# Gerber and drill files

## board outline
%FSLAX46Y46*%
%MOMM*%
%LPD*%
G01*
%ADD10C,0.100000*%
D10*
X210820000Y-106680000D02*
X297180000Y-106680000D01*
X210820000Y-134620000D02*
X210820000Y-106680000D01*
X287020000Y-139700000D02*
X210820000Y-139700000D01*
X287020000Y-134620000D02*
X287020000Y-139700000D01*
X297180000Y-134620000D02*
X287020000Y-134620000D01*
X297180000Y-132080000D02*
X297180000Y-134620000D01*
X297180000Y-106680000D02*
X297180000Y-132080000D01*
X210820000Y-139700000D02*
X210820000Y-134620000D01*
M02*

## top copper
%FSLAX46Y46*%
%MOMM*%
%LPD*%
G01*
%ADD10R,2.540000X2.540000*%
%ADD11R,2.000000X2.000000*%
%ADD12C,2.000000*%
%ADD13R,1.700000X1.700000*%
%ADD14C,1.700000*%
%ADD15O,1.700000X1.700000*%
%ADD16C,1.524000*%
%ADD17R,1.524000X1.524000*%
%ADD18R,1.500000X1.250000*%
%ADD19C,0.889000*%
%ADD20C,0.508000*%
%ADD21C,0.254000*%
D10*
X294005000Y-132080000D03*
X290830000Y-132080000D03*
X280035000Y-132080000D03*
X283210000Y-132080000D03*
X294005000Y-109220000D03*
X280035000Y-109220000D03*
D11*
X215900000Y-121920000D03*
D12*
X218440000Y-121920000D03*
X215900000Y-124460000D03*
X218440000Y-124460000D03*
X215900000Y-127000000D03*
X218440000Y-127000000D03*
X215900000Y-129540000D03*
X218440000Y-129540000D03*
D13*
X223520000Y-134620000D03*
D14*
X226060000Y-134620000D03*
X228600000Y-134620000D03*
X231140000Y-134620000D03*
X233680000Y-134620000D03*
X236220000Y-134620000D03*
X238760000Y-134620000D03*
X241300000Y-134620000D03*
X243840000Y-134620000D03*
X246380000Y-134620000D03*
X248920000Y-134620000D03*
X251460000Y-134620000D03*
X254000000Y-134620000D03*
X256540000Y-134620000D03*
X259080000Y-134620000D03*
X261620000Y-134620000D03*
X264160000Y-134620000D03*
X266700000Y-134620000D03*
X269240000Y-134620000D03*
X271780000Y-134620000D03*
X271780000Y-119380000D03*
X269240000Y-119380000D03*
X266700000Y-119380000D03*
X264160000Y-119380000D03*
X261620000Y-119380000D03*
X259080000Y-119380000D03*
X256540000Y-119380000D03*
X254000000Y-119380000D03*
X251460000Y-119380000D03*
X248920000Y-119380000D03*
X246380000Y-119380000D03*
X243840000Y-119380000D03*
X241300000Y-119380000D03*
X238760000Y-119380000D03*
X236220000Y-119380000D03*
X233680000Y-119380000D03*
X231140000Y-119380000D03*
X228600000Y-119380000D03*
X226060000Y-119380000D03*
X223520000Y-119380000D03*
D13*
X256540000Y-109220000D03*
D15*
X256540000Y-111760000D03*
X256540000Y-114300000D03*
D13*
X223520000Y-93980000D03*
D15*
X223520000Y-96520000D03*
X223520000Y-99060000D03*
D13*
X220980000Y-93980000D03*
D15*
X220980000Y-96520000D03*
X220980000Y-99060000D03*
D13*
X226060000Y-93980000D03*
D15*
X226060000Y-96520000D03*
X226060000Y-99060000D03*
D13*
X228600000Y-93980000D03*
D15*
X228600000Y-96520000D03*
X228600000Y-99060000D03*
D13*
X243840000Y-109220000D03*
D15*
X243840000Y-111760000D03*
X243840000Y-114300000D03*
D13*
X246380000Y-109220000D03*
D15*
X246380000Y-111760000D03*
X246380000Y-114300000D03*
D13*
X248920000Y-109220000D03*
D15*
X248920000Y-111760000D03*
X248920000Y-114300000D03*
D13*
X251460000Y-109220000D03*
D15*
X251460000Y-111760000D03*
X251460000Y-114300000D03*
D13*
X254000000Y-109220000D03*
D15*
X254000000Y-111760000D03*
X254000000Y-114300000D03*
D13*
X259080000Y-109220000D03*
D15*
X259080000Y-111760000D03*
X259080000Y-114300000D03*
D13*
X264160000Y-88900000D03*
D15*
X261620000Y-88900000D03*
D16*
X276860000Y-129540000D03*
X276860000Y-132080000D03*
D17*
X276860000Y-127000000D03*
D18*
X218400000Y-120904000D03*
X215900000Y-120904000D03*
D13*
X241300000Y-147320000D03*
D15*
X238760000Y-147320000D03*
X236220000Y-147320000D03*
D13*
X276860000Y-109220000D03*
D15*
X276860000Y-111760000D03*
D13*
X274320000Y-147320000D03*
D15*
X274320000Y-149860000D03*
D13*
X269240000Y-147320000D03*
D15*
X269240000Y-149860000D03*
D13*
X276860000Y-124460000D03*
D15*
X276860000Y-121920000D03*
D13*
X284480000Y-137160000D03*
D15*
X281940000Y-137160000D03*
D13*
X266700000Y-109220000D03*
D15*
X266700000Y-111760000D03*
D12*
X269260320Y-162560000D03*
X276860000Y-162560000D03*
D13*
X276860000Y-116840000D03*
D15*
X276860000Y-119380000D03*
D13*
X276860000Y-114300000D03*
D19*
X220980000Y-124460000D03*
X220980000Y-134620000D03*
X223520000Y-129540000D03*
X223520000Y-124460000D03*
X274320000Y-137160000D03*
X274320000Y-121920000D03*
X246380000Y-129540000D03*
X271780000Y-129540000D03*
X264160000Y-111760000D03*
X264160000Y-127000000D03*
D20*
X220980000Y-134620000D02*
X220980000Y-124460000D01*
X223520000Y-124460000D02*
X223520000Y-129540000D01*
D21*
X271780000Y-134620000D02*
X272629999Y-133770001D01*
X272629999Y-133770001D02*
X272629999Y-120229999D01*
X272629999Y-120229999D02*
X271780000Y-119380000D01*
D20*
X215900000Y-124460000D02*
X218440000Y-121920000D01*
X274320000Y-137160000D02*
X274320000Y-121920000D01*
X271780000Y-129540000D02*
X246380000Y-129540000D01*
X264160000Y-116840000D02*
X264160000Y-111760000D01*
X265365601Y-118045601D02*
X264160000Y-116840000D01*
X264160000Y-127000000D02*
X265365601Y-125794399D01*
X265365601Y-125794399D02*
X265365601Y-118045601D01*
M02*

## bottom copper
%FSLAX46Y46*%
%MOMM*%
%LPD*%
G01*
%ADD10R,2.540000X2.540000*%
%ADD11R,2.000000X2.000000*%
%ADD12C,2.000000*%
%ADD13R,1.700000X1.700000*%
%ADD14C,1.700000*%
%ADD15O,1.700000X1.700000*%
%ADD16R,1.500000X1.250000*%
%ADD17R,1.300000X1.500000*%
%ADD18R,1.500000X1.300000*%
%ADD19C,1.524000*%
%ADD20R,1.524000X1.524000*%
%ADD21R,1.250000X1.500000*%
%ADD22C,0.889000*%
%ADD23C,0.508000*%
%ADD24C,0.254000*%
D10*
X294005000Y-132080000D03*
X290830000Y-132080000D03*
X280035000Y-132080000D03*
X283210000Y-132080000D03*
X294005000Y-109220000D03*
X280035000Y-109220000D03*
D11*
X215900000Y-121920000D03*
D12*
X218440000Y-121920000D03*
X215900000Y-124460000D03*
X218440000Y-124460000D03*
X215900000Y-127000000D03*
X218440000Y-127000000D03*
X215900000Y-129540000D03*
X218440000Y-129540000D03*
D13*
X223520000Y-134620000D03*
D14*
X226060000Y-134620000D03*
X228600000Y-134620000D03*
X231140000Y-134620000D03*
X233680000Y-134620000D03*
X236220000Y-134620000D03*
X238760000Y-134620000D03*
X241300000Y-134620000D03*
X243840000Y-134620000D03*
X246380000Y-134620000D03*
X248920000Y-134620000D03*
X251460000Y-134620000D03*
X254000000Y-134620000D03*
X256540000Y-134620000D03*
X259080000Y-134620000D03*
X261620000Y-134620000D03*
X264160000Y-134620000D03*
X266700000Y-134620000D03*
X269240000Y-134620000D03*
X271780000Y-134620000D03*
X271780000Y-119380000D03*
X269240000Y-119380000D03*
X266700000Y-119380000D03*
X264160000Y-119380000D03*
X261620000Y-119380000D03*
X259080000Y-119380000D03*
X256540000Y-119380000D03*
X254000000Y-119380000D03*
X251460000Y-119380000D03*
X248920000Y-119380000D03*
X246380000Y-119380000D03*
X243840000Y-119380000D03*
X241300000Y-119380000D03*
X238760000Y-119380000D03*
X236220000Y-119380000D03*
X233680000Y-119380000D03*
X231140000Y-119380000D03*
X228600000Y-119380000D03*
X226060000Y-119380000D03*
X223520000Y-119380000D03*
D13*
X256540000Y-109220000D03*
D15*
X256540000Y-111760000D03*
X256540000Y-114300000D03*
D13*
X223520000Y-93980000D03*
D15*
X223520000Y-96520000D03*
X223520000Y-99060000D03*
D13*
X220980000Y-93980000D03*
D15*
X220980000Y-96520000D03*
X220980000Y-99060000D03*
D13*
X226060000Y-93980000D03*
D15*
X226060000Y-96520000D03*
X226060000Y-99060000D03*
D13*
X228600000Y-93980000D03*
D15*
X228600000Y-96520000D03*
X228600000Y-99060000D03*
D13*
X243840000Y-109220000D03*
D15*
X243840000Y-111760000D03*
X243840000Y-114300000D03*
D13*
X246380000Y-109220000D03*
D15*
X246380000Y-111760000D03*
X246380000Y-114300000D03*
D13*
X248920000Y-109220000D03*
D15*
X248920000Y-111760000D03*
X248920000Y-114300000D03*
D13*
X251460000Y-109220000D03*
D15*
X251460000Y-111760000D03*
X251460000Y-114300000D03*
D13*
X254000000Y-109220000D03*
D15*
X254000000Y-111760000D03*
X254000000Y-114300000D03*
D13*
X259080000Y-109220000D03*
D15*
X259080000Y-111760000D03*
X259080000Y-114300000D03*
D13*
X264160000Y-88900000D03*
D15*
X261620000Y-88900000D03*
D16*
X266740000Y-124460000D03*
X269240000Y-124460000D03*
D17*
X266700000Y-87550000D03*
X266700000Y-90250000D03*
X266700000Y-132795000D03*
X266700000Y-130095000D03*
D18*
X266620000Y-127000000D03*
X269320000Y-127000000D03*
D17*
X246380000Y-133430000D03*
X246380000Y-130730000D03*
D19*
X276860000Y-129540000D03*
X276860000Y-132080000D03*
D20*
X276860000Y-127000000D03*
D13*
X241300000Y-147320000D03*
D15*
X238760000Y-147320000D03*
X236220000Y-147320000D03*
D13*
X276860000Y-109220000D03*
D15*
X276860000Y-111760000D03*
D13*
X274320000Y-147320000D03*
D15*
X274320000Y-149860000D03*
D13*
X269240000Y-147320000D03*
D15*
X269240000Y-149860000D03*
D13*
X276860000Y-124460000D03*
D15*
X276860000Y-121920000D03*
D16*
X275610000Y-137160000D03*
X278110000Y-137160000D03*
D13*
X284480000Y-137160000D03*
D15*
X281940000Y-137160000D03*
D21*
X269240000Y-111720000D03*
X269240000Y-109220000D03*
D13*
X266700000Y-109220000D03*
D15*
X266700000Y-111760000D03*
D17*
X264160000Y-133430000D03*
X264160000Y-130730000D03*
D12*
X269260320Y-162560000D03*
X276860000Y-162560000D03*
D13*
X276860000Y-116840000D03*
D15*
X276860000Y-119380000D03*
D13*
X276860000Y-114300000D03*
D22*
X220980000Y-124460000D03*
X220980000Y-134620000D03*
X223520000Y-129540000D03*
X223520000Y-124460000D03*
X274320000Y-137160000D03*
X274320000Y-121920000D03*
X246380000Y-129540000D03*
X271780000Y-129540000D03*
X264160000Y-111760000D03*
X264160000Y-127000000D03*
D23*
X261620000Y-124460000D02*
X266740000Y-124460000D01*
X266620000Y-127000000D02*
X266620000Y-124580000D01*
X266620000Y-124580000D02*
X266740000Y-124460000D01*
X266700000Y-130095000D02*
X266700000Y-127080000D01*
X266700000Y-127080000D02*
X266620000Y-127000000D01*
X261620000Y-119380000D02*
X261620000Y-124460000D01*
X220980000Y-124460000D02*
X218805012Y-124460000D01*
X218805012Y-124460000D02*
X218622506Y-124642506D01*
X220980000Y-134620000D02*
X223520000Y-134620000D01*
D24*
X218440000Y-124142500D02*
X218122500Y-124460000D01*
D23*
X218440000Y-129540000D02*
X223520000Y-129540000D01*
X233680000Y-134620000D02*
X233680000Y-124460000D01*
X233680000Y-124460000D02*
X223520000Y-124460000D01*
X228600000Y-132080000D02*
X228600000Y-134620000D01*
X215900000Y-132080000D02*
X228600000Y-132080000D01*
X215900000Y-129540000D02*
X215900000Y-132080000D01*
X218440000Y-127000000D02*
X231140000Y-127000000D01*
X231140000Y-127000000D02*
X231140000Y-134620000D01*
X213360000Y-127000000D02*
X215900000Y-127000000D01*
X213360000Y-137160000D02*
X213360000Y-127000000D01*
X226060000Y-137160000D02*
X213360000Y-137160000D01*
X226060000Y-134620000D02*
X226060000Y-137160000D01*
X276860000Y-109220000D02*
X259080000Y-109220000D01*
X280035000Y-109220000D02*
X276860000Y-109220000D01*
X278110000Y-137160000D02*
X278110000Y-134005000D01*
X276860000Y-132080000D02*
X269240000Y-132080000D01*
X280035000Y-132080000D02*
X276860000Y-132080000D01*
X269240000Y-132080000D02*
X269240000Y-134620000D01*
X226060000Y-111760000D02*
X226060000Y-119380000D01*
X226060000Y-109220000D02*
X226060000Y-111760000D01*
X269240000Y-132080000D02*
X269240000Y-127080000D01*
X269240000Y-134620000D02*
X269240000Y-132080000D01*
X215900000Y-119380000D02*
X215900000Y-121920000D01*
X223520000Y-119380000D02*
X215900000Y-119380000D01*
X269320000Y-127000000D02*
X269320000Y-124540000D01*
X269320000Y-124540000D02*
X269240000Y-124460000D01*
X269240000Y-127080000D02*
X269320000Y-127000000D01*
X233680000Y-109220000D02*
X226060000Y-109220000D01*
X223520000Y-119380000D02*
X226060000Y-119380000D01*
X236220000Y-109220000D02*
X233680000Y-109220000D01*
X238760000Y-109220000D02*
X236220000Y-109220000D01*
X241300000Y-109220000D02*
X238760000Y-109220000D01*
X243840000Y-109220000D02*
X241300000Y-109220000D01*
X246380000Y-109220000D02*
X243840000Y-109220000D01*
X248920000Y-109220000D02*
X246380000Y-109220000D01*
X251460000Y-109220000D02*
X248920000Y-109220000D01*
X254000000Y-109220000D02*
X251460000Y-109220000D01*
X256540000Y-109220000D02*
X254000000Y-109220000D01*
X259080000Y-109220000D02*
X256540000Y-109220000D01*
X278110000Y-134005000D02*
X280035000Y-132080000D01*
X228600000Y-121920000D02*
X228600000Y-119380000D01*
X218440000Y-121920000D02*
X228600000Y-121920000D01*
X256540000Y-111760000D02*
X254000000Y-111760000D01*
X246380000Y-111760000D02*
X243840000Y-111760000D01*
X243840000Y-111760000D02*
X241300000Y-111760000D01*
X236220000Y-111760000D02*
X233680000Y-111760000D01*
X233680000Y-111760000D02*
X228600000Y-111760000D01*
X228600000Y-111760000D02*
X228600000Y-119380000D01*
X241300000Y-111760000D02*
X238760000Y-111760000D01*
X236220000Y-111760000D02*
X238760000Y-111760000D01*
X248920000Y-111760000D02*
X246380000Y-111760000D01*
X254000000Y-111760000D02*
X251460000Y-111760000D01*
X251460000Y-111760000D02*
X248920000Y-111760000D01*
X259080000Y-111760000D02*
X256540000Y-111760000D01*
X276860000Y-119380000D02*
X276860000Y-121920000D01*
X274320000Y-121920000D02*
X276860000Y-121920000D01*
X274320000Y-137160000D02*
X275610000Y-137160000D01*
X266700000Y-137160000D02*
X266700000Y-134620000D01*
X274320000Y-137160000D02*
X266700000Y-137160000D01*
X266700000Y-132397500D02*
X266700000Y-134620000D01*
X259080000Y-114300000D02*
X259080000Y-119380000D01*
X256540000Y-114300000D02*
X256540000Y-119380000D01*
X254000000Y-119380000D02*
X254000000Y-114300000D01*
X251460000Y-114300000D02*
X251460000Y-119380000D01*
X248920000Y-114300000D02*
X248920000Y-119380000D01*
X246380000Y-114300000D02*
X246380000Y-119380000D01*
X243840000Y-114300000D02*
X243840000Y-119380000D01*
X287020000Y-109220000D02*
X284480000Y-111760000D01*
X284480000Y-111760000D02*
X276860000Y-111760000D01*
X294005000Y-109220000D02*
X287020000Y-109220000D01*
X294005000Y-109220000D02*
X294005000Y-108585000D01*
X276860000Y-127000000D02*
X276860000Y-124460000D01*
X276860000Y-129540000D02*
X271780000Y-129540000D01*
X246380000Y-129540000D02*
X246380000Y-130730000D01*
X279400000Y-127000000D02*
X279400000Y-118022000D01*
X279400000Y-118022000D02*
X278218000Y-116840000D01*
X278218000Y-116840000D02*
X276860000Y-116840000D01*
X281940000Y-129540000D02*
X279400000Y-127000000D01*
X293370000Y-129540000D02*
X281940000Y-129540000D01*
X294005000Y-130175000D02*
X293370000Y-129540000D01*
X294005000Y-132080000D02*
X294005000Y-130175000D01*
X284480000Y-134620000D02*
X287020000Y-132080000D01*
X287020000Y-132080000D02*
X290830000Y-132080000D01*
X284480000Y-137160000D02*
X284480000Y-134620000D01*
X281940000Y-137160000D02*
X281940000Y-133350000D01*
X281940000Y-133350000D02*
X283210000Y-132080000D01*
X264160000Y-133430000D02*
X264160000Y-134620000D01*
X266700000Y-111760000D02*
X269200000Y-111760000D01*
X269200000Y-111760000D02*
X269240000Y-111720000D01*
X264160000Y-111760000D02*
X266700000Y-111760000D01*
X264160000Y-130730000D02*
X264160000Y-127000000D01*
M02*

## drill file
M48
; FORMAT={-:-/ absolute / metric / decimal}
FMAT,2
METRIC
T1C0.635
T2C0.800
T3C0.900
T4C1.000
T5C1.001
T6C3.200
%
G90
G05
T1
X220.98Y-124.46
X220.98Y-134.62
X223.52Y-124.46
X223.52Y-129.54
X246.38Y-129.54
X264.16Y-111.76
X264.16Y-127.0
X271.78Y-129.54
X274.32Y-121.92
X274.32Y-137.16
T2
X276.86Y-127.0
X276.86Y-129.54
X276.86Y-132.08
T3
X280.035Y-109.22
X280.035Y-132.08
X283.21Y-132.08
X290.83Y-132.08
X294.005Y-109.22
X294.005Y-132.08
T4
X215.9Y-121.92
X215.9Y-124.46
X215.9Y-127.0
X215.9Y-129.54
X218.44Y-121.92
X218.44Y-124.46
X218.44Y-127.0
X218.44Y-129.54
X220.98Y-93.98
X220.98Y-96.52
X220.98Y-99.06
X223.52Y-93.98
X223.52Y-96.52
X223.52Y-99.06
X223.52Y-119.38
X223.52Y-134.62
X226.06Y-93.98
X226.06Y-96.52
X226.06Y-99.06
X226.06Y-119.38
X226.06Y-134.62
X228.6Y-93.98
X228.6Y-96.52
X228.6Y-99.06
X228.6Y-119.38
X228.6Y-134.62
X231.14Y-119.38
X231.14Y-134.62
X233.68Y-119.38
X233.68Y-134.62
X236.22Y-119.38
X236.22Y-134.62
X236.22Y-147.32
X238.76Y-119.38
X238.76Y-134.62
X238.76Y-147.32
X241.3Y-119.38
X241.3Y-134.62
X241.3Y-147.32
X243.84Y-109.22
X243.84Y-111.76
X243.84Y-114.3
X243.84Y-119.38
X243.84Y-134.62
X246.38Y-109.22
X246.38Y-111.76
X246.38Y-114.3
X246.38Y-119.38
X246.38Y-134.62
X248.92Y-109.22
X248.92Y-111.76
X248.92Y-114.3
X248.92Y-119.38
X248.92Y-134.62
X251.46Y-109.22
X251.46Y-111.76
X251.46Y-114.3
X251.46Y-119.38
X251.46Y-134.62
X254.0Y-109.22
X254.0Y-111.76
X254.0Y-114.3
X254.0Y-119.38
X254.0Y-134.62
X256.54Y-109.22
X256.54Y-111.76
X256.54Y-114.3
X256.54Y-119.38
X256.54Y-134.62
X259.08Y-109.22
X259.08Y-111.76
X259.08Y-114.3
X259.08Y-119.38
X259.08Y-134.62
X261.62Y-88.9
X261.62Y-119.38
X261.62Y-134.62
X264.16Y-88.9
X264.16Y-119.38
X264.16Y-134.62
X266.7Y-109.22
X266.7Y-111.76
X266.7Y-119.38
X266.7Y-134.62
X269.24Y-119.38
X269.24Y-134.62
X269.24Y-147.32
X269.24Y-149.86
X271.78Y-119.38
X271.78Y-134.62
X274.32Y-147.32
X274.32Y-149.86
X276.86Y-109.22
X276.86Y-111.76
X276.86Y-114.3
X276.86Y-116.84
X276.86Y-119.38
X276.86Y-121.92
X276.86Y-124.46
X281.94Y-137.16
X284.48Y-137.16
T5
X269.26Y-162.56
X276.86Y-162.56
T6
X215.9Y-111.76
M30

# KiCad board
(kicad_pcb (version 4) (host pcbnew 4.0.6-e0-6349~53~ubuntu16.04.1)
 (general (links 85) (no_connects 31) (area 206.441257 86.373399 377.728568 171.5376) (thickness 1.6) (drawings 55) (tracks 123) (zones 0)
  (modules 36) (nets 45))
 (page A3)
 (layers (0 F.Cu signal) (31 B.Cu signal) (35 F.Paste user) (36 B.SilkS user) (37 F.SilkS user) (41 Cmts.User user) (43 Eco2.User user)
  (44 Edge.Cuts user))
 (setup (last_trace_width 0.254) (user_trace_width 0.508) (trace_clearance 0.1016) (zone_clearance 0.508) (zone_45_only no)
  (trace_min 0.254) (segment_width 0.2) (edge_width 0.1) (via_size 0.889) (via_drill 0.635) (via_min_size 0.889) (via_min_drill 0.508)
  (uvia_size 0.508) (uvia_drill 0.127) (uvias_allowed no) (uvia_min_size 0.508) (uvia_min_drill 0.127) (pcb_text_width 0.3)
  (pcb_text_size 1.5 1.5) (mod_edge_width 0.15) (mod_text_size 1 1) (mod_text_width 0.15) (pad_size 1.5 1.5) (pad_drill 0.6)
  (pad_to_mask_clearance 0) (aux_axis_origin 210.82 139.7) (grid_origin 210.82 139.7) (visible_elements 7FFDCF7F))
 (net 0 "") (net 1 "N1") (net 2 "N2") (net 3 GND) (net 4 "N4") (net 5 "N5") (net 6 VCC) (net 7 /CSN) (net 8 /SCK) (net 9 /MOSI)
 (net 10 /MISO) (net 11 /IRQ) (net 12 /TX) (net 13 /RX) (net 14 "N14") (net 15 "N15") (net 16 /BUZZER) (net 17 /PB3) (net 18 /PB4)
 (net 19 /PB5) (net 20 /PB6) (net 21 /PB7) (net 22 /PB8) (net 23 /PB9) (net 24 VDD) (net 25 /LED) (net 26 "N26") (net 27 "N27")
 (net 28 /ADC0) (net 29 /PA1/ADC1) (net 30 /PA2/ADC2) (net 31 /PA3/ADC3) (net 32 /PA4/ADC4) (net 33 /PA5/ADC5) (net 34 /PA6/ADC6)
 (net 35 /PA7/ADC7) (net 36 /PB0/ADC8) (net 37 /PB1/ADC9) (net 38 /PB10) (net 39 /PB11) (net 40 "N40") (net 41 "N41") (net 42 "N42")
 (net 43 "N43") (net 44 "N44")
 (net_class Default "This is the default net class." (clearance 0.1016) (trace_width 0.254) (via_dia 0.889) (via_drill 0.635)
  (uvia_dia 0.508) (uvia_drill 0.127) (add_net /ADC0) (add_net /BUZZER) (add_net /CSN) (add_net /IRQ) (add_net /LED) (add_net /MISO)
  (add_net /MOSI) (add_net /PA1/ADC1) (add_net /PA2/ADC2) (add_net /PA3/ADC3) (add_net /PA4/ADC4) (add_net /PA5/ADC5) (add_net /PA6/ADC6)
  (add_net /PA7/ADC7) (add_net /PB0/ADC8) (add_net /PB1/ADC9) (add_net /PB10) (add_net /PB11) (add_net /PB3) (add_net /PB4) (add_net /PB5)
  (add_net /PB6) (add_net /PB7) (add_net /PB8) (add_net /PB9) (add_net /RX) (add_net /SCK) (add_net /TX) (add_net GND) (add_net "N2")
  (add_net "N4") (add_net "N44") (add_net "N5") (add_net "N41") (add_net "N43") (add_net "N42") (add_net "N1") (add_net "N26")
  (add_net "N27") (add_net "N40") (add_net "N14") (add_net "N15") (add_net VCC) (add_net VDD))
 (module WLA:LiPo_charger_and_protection (layer F.Cu) (at 287.02 120.65 270)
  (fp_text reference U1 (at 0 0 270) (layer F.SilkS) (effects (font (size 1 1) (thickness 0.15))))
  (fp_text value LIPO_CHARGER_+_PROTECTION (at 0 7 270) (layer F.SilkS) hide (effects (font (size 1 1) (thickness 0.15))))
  (pad 3 thru_hole rect (at 11.43 -6.985 270) (size 2.54 2.54) (drill 0.9) (layers *.Cu *.Mask F.SilkS) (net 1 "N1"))
  (pad 1 thru_hole rect (at 11.43 -3.81 270) (size 2.54 2.54) (drill 0.9) (layers *.Cu *.Mask F.SilkS) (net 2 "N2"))
  (pad 4 thru_hole rect (at 11.43 6.985 270) (size 2.54 2.54) (drill 0.9) (layers *.Cu *.Mask F.SilkS) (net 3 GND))
  (pad 2 thru_hole rect (at 11.43 3.81 270) (size 2.54 2.54) (drill 0.9) (layers *.Cu *.Mask F.SilkS) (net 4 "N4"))
  (pad 5 thru_hole rect (at -11.43 -6.985 270) (size 2.54 2.54) (drill 0.9) (layers *.Cu *.Mask F.SilkS) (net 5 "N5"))
  (pad 6 thru_hole rect (at -11.43 6.985 270) (size 2.54 2.54) (drill 0.9) (layers *.Cu *.Mask F.SilkS) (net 3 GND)))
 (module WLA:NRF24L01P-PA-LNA (layer F.Cu) (at 215.9 125.73 270)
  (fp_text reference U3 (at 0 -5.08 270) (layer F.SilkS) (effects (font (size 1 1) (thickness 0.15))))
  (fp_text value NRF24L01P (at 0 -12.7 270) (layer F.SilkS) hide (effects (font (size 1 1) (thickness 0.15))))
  (pad 1 thru_hole rect (at -3.81 0 270) (size 2 2) (drill 1) (layers *.Cu *.Mask F.SilkS) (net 3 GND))
  (pad 2 thru_hole circle (at -3.81 -2.54 270) (size 2 2) (drill 1) (layers *.Cu *.Mask F.SilkS) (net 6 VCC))
  (pad 3 thru_hole circle (at -1.27 0 270) (size 2 2) (drill 1) (layers *.Cu *.Mask F.SilkS) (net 6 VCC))
  (pad 4 thru_hole circle (at -1.27 -2.54 270) (size 2 2) (drill 1) (layers *.Cu *.Mask F.SilkS) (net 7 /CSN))
  (pad 5 thru_hole circle (at 1.27 0 270) (size 2 2) (drill 1) (layers *.Cu *.Mask F.SilkS) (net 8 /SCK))
  (pad 6 thru_hole circle (at 1.27 -2.54 270) (size 2 2) (drill 1) (layers *.Cu *.Mask F.SilkS) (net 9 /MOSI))
  (pad 7 thru_hole circle (at 3.81 0 270) (size 2 2) (drill 1) (layers *.Cu *.Mask F.SilkS) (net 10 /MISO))
  (pad 8 thru_hole circle (at 3.81 -2.54 270) (size 2 2) (drill 1) (layers *.Cu *.Mask F.SilkS) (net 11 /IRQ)))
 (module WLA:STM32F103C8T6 (layer F.Cu) (at 247.65 127)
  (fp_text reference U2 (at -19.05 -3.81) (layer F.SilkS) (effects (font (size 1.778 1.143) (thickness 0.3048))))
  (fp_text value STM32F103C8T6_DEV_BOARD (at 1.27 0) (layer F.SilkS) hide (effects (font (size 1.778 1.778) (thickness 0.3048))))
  (pad 1 thru_hole rect (at -24.13 7.62) (size 1.7 1.7) (drill 1) (layers *.Cu *.Mask F.SilkS) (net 7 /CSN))
  (pad 2 thru_hole circle (at -21.59 7.62) (size 1.7 1.7) (drill 1) (layers *.Cu *.Mask F.SilkS) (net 8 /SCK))
  (pad 3 thru_hole circle (at -19.05 7.62) (size 1.7 1.7) (drill 1) (layers *.Cu *.Mask F.SilkS) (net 10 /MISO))
  (pad 4 thru_hole circle (at -16.51 7.62) (size 1.7 1.7) (drill 1) (layers *.Cu *.Mask F.SilkS) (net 9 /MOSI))
  (pad 5 thru_hole circle (at -13.97 7.62) (size 1.7 1.7) (drill 1) (layers *.Cu *.Mask F.SilkS) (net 11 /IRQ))
  (pad 6 thru_hole circle (at -11.43 7.62) (size 1.7 1.7) (drill 1) (layers *.Cu *.Mask F.SilkS) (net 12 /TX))
  (pad 7 thru_hole circle (at -8.89 7.62) (size 1.7 1.7) (drill 1) (layers *.Cu *.Mask F.SilkS) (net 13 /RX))
  (pad 8 thru_hole circle (at -6.35 7.62) (size 1.7 1.7) (drill 1) (layers *.Cu *.Mask F.SilkS) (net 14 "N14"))
  (pad 9 thru_hole circle (at -3.81 7.62) (size 1.7 1.7) (drill 1) (layers *.Cu *.Mask F.SilkS) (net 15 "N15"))
  (pad 10 thru_hole circle (at -1.27 7.62) (size 1.7 1.7) (drill 1) (layers *.Cu *.Mask F.SilkS) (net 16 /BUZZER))
  (pad 11 thru_hole circle (at 1.27 7.62) (size 1.7 1.7) (drill 1) (layers *.Cu *.Mask F.SilkS) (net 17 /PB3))
  (pad 12 thru_hole circle (at 3.81 7.62) (size 1.7 1.7) (drill 1) (layers *.Cu *.Mask F.SilkS) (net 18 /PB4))
  (pad 13 thru_hole circle (at 6.35 7.62) (size 1.7 1.7) (drill 1) (layers *.Cu *.Mask F.SilkS) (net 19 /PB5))
  (pad 14 thru_hole circle (at 8.89 7.62) (size 1.7 1.7) (drill 1) (layers *.Cu *.Mask F.SilkS) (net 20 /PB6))
  (pad 15 thru_hole circle (at 11.43 7.62) (size 1.7 1.7) (drill 1) (layers *.Cu *.Mask F.SilkS) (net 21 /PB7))
  (pad 16 thru_hole circle (at 13.97 7.62) (size 1.7 1.7) (drill 1) (layers *.Cu *.Mask F.SilkS) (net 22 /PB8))
  (pad 17 thru_hole circle (at 16.51 7.62) (size 1.7 1.7) (drill 1) (layers *.Cu *.Mask F.SilkS) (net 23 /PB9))
  (pad 18 thru_hole circle (at 19.05 7.62) (size 1.7 1.7) (drill 1) (layers *.Cu *.Mask F.SilkS) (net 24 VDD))
  (pad 19 thru_hole circle (at 21.59 7.62) (size 1.7 1.7) (drill 1) (layers *.Cu *.Mask F.SilkS) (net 3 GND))
  (pad 20 thru_hole circle (at 24.13 7.62) (size 1.7 1.7) (drill 1) (layers *.Cu *.Mask F.SilkS) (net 6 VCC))
  (pad 21 thru_hole circle (at 24.13 -7.62) (size 1.7 1.7) (drill 1) (layers *.Cu *.Mask F.SilkS) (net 6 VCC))
  (pad 22 thru_hole circle (at 21.59 -7.62) (size 1.7 1.7) (drill 1) (layers *.Cu *.Mask F.SilkS) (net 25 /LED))
  (pad 23 thru_hole circle (at 19.05 -7.62) (size 1.7 1.7) (drill 1) (layers *.Cu *.Mask F.SilkS) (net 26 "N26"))
  (pad 24 thru_hole circle (at 16.51 -7.62) (size 1.7 1.7) (drill 1) (layers *.Cu *.Mask F.SilkS) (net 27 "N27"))
  (pad 25 thru_hole circle (at 13.97 -7.62) (size 1.7 1.7) (drill 1) (layers *.Cu *.Mask F.SilkS) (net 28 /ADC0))
  (pad 26 thru_hole circle (at 11.43 -7.62) (size 1.7 1.7) (drill 1) (layers *.Cu *.Mask F.SilkS) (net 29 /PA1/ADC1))
  (pad 27 thru_hole circle (at 8.89 -7.62) (size 1.7 1.7) (drill 1) (layers *.Cu *.Mask F.SilkS) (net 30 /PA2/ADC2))
  (pad 28 thru_hole circle (at 6.35 -7.62) (size 1.7 1.7) (drill 1) (layers *.Cu *.Mask F.SilkS) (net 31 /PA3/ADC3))
  (pad 29 thru_hole circle (at 3.81 -7.62) (size 1.7 1.7) (drill 1) (layers *.Cu *.Mask F.SilkS) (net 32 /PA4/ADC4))
  (pad 30 thru_hole circle (at 1.27 -7.62) (size 1.7 1.7) (drill 1) (layers *.Cu *.Mask F.SilkS) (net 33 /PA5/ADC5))
  (pad 31 thru_hole circle (at -1.27 -7.62) (size 1.7 1.7) (drill 1) (layers *.Cu *.Mask F.SilkS) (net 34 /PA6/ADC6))
  (pad 32 thru_hole circle (at -3.81 -7.62) (size 1.7 1.7) (drill 1) (layers *.Cu *.Mask F.SilkS) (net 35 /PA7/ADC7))
  (pad 33 thru_hole circle (at -6.35 -7.62) (size 1.7 1.7) (drill 1) (layers *.Cu *.Mask F.SilkS) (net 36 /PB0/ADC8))
  (pad 34 thru_hole circle (at -8.89 -7.62) (size 1.7 1.7) (drill 1) (layers *.Cu *.Mask F.SilkS) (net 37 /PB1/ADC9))
  (pad 35 thru_hole circle (at -11.43 -7.62) (size 1.7 1.7) (drill 1) (layers *.Cu *.Mask F.SilkS) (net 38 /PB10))
  (pad 36 thru_hole circle (at -13.97 -7.62) (size 1.7 1.7) (drill 1) (layers *.Cu *.Mask F.SilkS) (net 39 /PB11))
  (pad 37 thru_hole circle (at -16.51 -7.62) (size 1.7 1.7) (drill 1) (layers *.Cu *.Mask F.SilkS) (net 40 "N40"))
  (pad 38 thru_hole circle (at -19.05 -7.62) (size 1.7 1.7) (drill 1) (layers *.Cu *.Mask F.SilkS) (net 6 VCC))
  (pad 39 thru_hole circle (at -21.59 -7.62) (size 1.7 1.7) (drill 1) (layers *.Cu *.Mask F.SilkS) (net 3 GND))
  (pad 40 thru_hole circle (at -24.13 -7.62) (size 1.7 1.7) (drill 1) (layers *.Cu *.Mask F.SilkS) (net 3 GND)))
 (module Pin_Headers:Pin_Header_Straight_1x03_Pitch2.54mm (layer F.Cu) (at 256.54 109.22)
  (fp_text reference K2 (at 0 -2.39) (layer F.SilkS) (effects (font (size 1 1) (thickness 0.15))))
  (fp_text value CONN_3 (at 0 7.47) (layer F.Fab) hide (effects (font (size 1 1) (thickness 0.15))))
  (pad 1 thru_hole rect (at 0 0) (size 1.7 1.7) (drill 1) (layers *.Cu *.Mask) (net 3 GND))
  (pad 2 thru_hole oval (at 0 2.54) (size 1.7 1.7) (drill 1) (layers *.Cu *.Mask) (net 6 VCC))
  (pad 3 thru_hole oval (at 0 5.08) (size 1.7 1.7) (drill 1) (layers *.Cu *.Mask) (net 30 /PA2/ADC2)))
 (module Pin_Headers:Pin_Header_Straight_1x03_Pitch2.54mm (layer F.Cu) (at 223.52 93.98)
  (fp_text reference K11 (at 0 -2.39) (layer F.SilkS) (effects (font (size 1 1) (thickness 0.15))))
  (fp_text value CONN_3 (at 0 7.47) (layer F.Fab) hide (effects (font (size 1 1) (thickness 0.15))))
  (pad 1 thru_hole rect (at 0 0) (size 1.7 1.7) (drill 1) (layers *.Cu *.Mask) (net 3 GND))
  (pad 2 thru_hole oval (at 0 2.54) (size 1.7 1.7) (drill 1) (layers *.Cu *.Mask) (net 6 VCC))
  (pad 3 thru_hole oval (at 0 5.08) (size 1.7 1.7) (drill 1) (layers *.Cu *.Mask) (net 38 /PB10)))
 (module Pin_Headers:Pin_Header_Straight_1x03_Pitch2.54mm (layer F.Cu) (at 220.98 93.98)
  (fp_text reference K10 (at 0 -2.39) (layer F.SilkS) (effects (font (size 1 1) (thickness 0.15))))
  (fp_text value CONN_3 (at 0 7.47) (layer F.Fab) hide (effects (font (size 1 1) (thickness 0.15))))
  (pad 1 thru_hole rect (at 0 0) (size 1.7 1.7) (drill 1) (layers *.Cu *.Mask) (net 3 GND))
  (pad 2 thru_hole oval (at 0 2.54) (size 1.7 1.7) (drill 1) (layers *.Cu *.Mask) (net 6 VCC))
  (pad 3 thru_hole oval (at 0 5.08) (size 1.7 1.7) (drill 1) (layers *.Cu *.Mask) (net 39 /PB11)))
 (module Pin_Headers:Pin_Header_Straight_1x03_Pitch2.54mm (layer F.Cu) (at 226.06 93.98)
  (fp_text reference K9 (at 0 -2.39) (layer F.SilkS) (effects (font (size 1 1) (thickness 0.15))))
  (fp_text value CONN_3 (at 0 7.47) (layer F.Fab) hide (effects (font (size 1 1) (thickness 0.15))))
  (pad 1 thru_hole rect (at 0 0) (size 1.7 1.7) (drill 1) (layers *.Cu *.Mask) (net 3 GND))
  (pad 2 thru_hole oval (at 0 2.54) (size 1.7 1.7) (drill 1) (layers *.Cu *.Mask) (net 6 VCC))
  (pad 3 thru_hole oval (at 0 5.08) (size 1.7 1.7) (drill 1) (layers *.Cu *.Mask) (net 37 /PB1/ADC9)))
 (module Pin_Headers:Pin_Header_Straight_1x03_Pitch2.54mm (layer F.Cu) (at 228.6 93.98)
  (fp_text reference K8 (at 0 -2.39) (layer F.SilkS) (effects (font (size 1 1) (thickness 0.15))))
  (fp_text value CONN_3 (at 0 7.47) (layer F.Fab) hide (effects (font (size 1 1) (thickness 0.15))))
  (pad 1 thru_hole rect (at 0 0) (size 1.7 1.7) (drill 1) (layers *.Cu *.Mask) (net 3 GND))
  (pad 2 thru_hole oval (at 0 2.54) (size 1.7 1.7) (drill 1) (layers *.Cu *.Mask) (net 6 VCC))
  (pad 3 thru_hole oval (at 0 5.08) (size 1.7 1.7) (drill 1) (layers *.Cu *.Mask) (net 36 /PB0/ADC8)))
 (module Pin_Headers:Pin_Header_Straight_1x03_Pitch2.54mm (layer F.Cu) (at 243.84 109.22)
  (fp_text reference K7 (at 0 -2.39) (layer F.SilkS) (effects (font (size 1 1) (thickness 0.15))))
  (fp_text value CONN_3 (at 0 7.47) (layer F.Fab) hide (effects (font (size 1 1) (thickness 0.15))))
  (pad 1 thru_hole rect (at 0 0) (size 1.7 1.7) (drill 1) (layers *.Cu *.Mask) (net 3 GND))
  (pad 2 thru_hole oval (at 0 2.54) (size 1.7 1.7) (drill 1) (layers *.Cu *.Mask) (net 6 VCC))
  (pad 3 thru_hole oval (at 0 5.08) (size 1.7 1.7) (drill 1) (layers *.Cu *.Mask) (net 35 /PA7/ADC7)))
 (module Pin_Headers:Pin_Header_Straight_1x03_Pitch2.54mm (layer F.Cu) (at 246.38 109.22)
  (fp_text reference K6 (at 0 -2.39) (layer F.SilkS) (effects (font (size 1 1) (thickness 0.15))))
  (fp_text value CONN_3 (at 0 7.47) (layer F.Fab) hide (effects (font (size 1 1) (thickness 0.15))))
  (pad 1 thru_hole rect (at 0 0) (size 1.7 1.7) (drill 1) (layers *.Cu *.Mask) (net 3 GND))
  (pad 2 thru_hole oval (at 0 2.54) (size 1.7 1.7) (drill 1) (layers *.Cu *.Mask) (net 6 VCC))
  (pad 3 thru_hole oval (at 0 5.08) (size 1.7 1.7) (drill 1) (layers *.Cu *.Mask) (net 34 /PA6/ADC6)))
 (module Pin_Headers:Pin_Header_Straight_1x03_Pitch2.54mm (layer F.Cu) (at 248.92 109.22)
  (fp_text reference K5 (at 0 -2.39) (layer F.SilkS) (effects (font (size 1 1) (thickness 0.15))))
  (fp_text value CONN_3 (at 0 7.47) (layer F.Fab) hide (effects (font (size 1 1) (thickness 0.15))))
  (pad 1 thru_hole rect (at 0 0) (size 1.7 1.7) (drill 1) (layers *.Cu *.Mask) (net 3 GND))
  (pad 2 thru_hole oval (at 0 2.54) (size 1.7 1.7) (drill 1) (layers *.Cu *.Mask) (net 6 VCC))
  (pad 3 thru_hole oval (at 0 5.08) (size 1.7 1.7) (drill 1) (layers *.Cu *.Mask) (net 33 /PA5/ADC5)))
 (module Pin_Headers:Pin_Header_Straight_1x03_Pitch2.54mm (layer F.Cu) (at 251.46 109.22)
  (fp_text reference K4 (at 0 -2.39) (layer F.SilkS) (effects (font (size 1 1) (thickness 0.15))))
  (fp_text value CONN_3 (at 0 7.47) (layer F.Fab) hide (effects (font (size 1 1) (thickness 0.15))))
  (pad 1 thru_hole rect (at 0 0) (size 1.7 1.7) (drill 1) (layers *.Cu *.Mask) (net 3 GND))
  (pad 2 thru_hole oval (at 0 2.54) (size 1.7 1.7) (drill 1) (layers *.Cu *.Mask) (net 6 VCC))
  (pad 3 thru_hole oval (at 0 5.08) (size 1.7 1.7) (drill 1) (layers *.Cu *.Mask) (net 32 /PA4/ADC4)))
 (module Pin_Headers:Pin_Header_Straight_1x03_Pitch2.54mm (layer F.Cu) (at 254 109.22)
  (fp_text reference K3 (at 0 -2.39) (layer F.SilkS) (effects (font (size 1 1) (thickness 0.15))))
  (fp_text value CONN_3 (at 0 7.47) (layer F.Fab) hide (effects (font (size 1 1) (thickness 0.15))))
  (pad 1 thru_hole rect (at 0 0) (size 1.7 1.7) (drill 1) (layers *.Cu *.Mask) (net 3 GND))
  (pad 2 thru_hole oval (at 0 2.54) (size 1.7 1.7) (drill 1) (layers *.Cu *.Mask) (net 6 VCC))
  (pad 3 thru_hole oval (at 0 5.08) (size 1.7 1.7) (drill 1) (layers *.Cu *.Mask) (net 31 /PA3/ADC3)))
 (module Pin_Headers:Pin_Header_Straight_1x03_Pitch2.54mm (layer F.Cu) (at 259.08 109.22)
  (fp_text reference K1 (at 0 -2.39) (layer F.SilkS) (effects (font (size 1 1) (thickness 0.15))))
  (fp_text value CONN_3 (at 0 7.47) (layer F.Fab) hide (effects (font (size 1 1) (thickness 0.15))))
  (pad 1 thru_hole rect (at 0 0) (size 1.7 1.7) (drill 1) (layers *.Cu *.Mask) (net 3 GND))
  (pad 2 thru_hole oval (at 0 2.54) (size 1.7 1.7) (drill 1) (layers *.Cu *.Mask) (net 6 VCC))
  (pad 3 thru_hole oval (at 0 5.08) (size 1.7 1.7) (drill 1) (layers *.Cu *.Mask) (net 29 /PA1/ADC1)))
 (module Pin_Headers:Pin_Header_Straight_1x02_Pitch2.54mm (layer F.Cu) (at 264.16 88.9 270)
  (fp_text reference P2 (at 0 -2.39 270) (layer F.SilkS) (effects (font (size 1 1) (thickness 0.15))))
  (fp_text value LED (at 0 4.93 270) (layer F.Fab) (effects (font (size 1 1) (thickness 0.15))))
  (pad 1 thru_hole rect (at 0 0 270) (size 1.7 1.7) (drill 1) (layers *.Cu *.Mask) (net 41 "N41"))
  (pad 2 thru_hole oval (at 0 2.54 270) (size 1.7 1.7) (drill 1) (layers *.Cu *.Mask) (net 6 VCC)))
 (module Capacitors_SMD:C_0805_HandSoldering (layer B.Cu) (at 267.99 124.46)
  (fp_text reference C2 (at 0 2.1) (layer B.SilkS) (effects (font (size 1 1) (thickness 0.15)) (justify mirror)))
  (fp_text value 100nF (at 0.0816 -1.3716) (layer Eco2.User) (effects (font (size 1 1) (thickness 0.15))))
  (pad 1 smd rect (at -1.25 0) (size 1.5 1.25) (layers B.Cu) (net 28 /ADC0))
  (pad 2 smd rect (at 1.25 0) (size 1.5 1.25) (layers B.Cu) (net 3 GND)))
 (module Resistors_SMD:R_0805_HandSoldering (layer B.Cu) (at 266.7 88.9 270)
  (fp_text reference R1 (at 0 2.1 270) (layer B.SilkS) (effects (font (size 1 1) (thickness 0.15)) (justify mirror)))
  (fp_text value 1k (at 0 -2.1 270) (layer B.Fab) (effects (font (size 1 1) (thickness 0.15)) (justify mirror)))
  (pad 1 smd rect (at -1.35 0 270) (size 1.5 1.3) (layers B.Cu) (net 41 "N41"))
  (pad 2 smd rect (at 1.35 0 270) (size 1.5 1.3) (layers B.Cu) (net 25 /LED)))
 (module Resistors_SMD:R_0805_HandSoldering (layer B.Cu) (at 266.7 131.445 90)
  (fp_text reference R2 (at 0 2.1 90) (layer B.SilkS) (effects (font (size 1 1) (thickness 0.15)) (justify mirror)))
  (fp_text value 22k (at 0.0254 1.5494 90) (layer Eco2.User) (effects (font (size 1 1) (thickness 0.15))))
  (pad 1 smd rect (at -1.35 0 90) (size 1.5 1.3) (layers B.Cu) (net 24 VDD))
  (pad 2 smd rect (at 1.35 0 90) (size 1.5 1.3) (layers B.Cu) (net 28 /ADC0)))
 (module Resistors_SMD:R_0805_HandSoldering (layer B.Cu) (at 267.97 127)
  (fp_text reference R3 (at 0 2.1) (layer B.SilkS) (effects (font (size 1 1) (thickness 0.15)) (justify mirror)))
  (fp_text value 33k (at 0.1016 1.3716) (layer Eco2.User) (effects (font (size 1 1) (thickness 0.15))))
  (pad 1 smd rect (at -1.35 0) (size 1.5 1.3) (layers B.Cu) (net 28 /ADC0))
  (pad 2 smd rect (at 1.35 0) (size 1.5 1.3) (layers B.Cu) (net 3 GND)))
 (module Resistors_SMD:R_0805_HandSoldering (layer B.Cu) (at 246.38 132.08 90)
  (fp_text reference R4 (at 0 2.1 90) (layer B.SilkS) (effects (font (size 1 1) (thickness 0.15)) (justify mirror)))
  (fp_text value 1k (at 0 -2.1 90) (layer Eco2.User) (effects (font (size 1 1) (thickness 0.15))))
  (pad 1 smd rect (at -1.35 0 90) (size 1.5 1.3) (layers B.Cu) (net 16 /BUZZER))
  (pad 2 smd rect (at 1.35 0 90) (size 1.5 1.3) (layers B.Cu) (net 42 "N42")))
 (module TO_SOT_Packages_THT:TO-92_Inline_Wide (layer F.Cu) (at 276.86 127 270)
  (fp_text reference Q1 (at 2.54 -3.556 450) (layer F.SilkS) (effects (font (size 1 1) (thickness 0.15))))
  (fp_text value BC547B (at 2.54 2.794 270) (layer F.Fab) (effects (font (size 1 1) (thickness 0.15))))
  (pad 2 thru_hole circle (at 2.54 0) (size 1.524 1.524) (drill 0.8) (layers *.Cu *.Mask) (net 42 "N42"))
  (pad 3 thru_hole circle (at 5.08 0) (size 1.524 1.524) (drill 0.8) (layers *.Cu *.Mask) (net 3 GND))
  (pad 1 thru_hole rect (at 0 0) (size 1.524 1.524) (drill 0.8) (layers *.Cu *.Mask) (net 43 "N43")))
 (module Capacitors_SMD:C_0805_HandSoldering (layer F.Cu) (at 217.15 120.904 180)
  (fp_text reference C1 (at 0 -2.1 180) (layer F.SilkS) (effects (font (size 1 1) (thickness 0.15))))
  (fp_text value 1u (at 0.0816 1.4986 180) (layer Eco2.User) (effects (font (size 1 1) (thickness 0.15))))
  (pad 1 smd rect (at -1.25 0 180) (size 1.5 1.25) (layers F.Cu F.Paste) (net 6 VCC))
  (pad 2 smd rect (at 1.25 0 180) (size 1.5 1.25) (layers F.Cu F.Paste) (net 3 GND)))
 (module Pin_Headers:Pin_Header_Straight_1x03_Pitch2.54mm (layer F.Cu) (at 241.3 147.32 270)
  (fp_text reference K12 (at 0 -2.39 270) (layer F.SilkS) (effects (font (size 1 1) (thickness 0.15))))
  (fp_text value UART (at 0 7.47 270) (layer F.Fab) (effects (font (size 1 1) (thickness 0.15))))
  (pad 1 thru_hole rect (at 0 0 270) (size 1.7 1.7) (drill 1) (layers *.Cu *.Mask) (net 3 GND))
  (pad 2 thru_hole oval (at 0 2.54 270) (size 1.7 1.7) (drill 1) (layers *.Cu *.Mask) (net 13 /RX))
  (pad 3 thru_hole oval (at 0 5.08 270) (size 1.7 1.7) (drill 1) (layers *.Cu *.Mask) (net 12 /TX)))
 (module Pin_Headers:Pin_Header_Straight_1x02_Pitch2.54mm (layer F.Cu) (at 276.86 109.22)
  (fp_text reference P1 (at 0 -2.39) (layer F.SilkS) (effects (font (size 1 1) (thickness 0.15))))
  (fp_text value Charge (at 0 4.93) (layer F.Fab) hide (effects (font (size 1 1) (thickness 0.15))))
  (pad 1 thru_hole rect (at 0 0) (size 1.7 1.7) (drill 1) (layers *.Cu *.Mask) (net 3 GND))
  (pad 2 thru_hole oval (at 0 2.54) (size 1.7 1.7) (drill 1) (layers *.Cu *.Mask) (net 5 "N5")))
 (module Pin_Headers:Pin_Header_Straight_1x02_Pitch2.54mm (layer F.Cu) (at 274.32 147.32)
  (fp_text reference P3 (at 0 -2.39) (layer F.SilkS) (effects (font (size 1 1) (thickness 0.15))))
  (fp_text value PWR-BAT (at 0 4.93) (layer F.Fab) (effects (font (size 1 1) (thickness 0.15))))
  (pad 1 thru_hole rect (at 0 0) (size 1.7 1.7) (drill 1) (layers *.Cu *.Mask) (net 3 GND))
  (pad 2 thru_hole oval (at 0 2.54) (size 1.7 1.7) (drill 1) (layers *.Cu *.Mask) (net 24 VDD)))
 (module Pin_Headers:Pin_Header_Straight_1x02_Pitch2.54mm (layer F.Cu) (at 269.24 147.32)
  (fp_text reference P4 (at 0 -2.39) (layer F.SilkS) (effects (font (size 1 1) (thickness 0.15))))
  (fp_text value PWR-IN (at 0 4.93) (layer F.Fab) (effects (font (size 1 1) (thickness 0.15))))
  (pad 1 thru_hole rect (at 0 0) (size 1.7 1.7) (drill 1) (layers *.Cu *.Mask) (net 3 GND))
  (pad 2 thru_hole oval (at 0 2.54) (size 1.7 1.7) (drill 1) (layers *.Cu *.Mask) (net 24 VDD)))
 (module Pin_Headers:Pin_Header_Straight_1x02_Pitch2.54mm (layer F.Cu) (at 276.86 124.46 180)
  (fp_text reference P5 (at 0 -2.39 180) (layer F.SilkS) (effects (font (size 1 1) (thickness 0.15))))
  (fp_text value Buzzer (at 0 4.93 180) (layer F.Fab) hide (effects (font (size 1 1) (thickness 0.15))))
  (pad 1 thru_hole rect (at 0 0 180) (size 1.7 1.7) (drill 1) (layers *.Cu *.Mask) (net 43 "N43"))
  (pad 2 thru_hole oval (at 0 2.54 180) (size 1.7 1.7) (drill 1) (layers *.Cu *.Mask) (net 24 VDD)))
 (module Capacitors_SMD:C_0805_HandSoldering (layer B.Cu) (at 276.86 137.16)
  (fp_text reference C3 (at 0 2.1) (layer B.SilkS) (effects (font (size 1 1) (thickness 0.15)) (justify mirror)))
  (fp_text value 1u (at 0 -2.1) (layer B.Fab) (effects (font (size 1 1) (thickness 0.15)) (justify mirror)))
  (pad 1 smd rect (at -1.25 0) (size 1.5 1.25) (layers B.Cu) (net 24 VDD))
  (pad 2 smd rect (at 1.25 0) (size 1.5 1.25) (layers B.Cu) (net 3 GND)))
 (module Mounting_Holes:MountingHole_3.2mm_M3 (layer F.Cu) (at 215.9 111.76)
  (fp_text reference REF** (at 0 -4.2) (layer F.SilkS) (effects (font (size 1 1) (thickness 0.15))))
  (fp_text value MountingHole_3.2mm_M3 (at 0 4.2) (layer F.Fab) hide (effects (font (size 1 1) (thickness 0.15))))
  (pad 1 np_thru_hole circle (at 0 0) (size 3.2 3.2) (drill 3.2) (layers *.Cu *.Mask)))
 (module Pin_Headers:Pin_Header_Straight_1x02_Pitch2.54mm (layer F.Cu) (at 284.48 137.16 270)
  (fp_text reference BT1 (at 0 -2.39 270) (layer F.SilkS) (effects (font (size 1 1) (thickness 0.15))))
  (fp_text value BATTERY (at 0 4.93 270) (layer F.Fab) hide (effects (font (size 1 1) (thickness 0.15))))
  (pad 1 thru_hole rect (at 0 0 270) (size 1.7 1.7) (drill 1) (layers *.Cu *.Mask) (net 2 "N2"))
  (pad 2 thru_hole oval (at 0 2.54 270) (size 1.7 1.7) (drill 1) (layers *.Cu *.Mask) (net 4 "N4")))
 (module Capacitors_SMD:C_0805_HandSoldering (layer B.Cu) (at 269.24 110.47 90)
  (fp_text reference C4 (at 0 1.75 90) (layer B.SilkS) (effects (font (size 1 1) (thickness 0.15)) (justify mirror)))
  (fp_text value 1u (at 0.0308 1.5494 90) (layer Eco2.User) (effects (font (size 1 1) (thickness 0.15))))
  (pad 1 smd rect (at -1.25 0 90) (size 1.5 1.25) (layers B.Cu) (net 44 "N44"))
  (pad 2 smd rect (at 1.25 0 90) (size 1.5 1.25) (layers B.Cu) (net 3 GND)))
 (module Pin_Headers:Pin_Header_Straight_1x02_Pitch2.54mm (layer F.Cu) (at 266.7 109.22)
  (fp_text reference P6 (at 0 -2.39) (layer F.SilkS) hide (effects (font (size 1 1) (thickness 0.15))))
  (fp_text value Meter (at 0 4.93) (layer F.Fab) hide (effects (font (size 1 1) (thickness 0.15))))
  (pad 1 thru_hole rect (at 0 0) (size 1.7 1.7) (drill 1) (layers *.Cu *.Mask) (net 3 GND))
  (pad 2 thru_hole oval (at 0 2.54) (size 1.7 1.7) (drill 1) (layers *.Cu *.Mask) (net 44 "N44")))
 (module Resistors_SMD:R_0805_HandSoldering (layer B.Cu) (at 264.16 132.08 90)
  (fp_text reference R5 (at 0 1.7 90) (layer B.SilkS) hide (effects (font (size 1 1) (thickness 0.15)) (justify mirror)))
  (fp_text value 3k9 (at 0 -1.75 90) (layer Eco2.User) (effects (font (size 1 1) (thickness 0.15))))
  (pad 1 smd rect (at -1.35 0 90) (size 1.5 1.3) (layers B.Cu) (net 23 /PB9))
  (pad 2 smd rect (at 1.35 0 90) (size 1.5 1.3) (layers B.Cu) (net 44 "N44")))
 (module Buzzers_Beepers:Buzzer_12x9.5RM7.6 (layer F.Cu) (at 273.06016 162.56)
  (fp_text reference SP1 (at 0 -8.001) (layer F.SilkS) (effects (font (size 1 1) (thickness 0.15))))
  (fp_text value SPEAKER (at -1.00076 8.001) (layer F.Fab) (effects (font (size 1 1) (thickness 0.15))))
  (pad 1 thru_hole circle (at -3.79984 0) (size 2 2) (drill 1.00076) (layers *.Cu *.Mask) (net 24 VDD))
  (pad 2 thru_hole circle (at 3.79984 0) (size 2 2) (drill 1.00076) (layers *.Cu *.Mask) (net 43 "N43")))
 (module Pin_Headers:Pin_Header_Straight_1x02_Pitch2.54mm (layer F.Cu) (at 276.86 116.84)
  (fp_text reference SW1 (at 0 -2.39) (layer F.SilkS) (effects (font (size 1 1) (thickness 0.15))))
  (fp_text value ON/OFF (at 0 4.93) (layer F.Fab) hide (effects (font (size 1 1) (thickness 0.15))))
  (pad 1 thru_hole rect (at 0 0) (size 1.7 1.7) (drill 1) (layers *.Cu *.Mask) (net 1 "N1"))
  (pad 2 thru_hole oval (at 0 2.54) (size 1.7 1.7) (drill 1) (layers *.Cu *.Mask) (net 24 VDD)))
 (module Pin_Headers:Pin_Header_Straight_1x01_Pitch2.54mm (layer F.Cu) (at 276.86 114.3)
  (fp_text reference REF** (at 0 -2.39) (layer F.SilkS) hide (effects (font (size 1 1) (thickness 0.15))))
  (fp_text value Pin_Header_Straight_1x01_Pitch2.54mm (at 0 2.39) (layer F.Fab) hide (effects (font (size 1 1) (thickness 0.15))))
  (pad 1 thru_hole rect (at 0 0) (size 1.7 1.7) (drill 1) (layers *.Cu *.Mask)))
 (gr_line (start 210.82 106.68) (end 297.18 106.68) (angle 90) (layer Edge.Cuts) (width 0.1))
 (gr_line (start 210.82 134.62) (end 210.82 106.68) (angle 90) (layer Edge.Cuts) (width 0.1))
 (gr_line (start 287.02 139.7) (end 210.82 139.7) (angle 90) (layer Edge.Cuts) (width 0.1))
 (gr_line (start 287.02 134.62) (end 287.02 139.7) (angle 90) (layer Edge.Cuts) (width 0.1))
 (gr_line (start 297.18 134.62) (end 287.02 134.62) (angle 90) (layer Edge.Cuts) (width 0.1))
 (gr_line (start 297.18 132.08) (end 297.18 134.62) (angle 90) (layer Edge.Cuts) (width 0.1))
 (gr_line (start 297.18 106.68) (end 297.18 132.08) (angle 90) (layer Edge.Cuts) (width 0.1))
 (gr_line (start 210.82 139.7) (end 210.82 134.62) (angle 90) (layer Edge.Cuts) (width 0.1))
 (segment (start 261.62 124.46) (end 266.74 124.46) (width 0.508) (layer B.Cu) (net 28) (status 20))
 (segment (start 266.62 127) (end 266.62 124.58) (width 0.508) (layer B.Cu) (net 28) (status 30))
 (segment (start 266.62 124.58) (end 266.74 124.46) (width 0.508) (layer B.Cu) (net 28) (status 30))
 (segment (start 266.7 130.095) (end 266.7 127.08) (width 0.508) (layer B.Cu) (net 28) (status 30))
 (segment (start 266.7 127.08) (end 266.62 127) (width 0.508) (layer B.Cu) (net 28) (status 30))
 (segment (start 261.62 119.38) (end 261.62 124.46) (width 0.508) (layer B.Cu) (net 28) (status 10))
 (segment (start 220.98 124.46) (end 218.805012 124.46) (width 0.508) (layer B.Cu) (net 7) (status 20))
 (segment (start 218.805012 124.46) (end 218.622506 124.642506) (width 0.508) (layer B.Cu) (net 7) (status 30))
 (segment (start 220.98 134.62) (end 220.98 124.46) (width 0.508) (layer F.Cu) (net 7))
 (via (at 220.98 124.46) (size 0.889) (drill 0.635) (layers F.Cu B.Cu) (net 7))
 (segment (start 220.98 134.62) (end 223.52 134.62) (width 0.508) (layer B.Cu) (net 7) (status 20))
 (via (at 220.98 134.62) (size 0.889) (drill 0.635) (layers F.Cu B.Cu) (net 7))
 (segment (start 218.44 124.1425) (end 218.1225 124.46) (width 0.254) (layer B.Cu) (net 7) (status 30))
 (segment (start 218.44 129.54) (end 223.52 129.54) (width 0.508) (layer B.Cu) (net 11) (status 10))
 (segment (start 223.52 124.46) (end 223.52 129.54) (width 0.508) (layer F.Cu) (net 11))
 (via (at 223.52 129.54) (size 0.889) (drill 0.635) (layers F.Cu B.Cu) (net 11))
 (segment (start 233.68 134.62) (end 233.68 124.46) (width 0.508) (layer B.Cu) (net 11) (status 10))
 (segment (start 233.68 124.46) (end 223.52 124.46) (width 0.508) (layer B.Cu) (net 11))
 (via (at 223.52 124.46) (size 0.889) (drill 0.635) (layers F.Cu B.Cu) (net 11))
 (segment (start 228.6 132.08) (end 228.6 134.62) (width 0.508) (layer B.Cu) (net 10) (status 20))
 (segment (start 215.9 132.08) (end 228.6 132.08) (width 0.508) (layer B.Cu) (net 10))
 (segment (start 215.9 129.54) (end 215.9 132.08) (width 0.508) (layer B.Cu) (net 10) (status 10))
 (segment (start 218.44 127) (end 231.14 127) (width 0.508) (layer B.Cu) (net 9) (status 10))
 (segment (start 231.14 127) (end 231.14 134.62) (width 0.508) (layer B.Cu) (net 9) (status 20))
 (segment (start 213.36 127) (end 215.9 127) (width 0.508) (layer B.Cu) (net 8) (status 20))
 (segment (start 213.36 137.16) (end 213.36 127) (width 0.508) (layer B.Cu) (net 8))
 (segment (start 226.06 137.16) (end 213.36 137.16) (width 0.508) (layer B.Cu) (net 8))
 (segment (start 226.06 134.62) (end 226.06 137.16) (width 0.508) (layer B.Cu) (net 8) (status 10))
 (segment (start 276.86 109.22) (end 259.08 109.22) (width 0.508) (layer B.Cu) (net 3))
 (segment (start 280.035 109.22) (end 276.86 109.22) (width 0.508) (layer B.Cu) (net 3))
 (segment (start 278.11 137.16) (end 278.11 134.005) (width 0.508) (layer B.Cu) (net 3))
 (segment (start 276.86 132.08) (end 269.24 132.08) (width 0.508) (layer B.Cu) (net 3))
 (segment (start 280.035 132.08) (end 276.86 132.08) (width 0.508) (layer B.Cu) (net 3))
 (segment (start 269.24 132.08) (end 269.24 134.62) (width 0.508) (layer B.Cu) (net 3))
 (segment (start 226.06 111.76) (end 226.06 119.38) (width 0.508) (layer B.Cu) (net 3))
 (segment (start 226.06 109.22) (end 226.06 111.76) (width 0.508) (layer B.Cu) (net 3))
 (segment (start 269.24 132.08) (end 269.24 127.08) (width 0.508) (layer B.Cu) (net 3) (status 20))
 (segment (start 269.24 134.62) (end 269.24 132.08) (width 0.508) (layer B.Cu) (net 3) (status 10))
 (segment (start 215.9 119.38) (end 215.9 121.92) (width 0.508) (layer B.Cu) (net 3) (status 20))
 (segment (start 223.52 119.38) (end 215.9 119.38) (width 0.508) (layer B.Cu) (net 3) (status 10))
 (segment (start 269.32 127) (end 269.32 124.54) (width 0.508) (layer B.Cu) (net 3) (status 30))
 (segment (start 269.32 124.54) (end 269.24 124.46) (width 0.508) (layer B.Cu) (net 3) (status 30))
 (segment (start 269.24 127.08) (end 269.32 127) (width 0.508) (layer B.Cu) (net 3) (status 30))
 (segment (start 233.68 109.22) (end 226.06 109.22) (width 0.508) (layer B.Cu) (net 3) (status 10))
 (segment (start 223.52 119.38) (end 226.06 119.38) (width 0.508) (layer B.Cu) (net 3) (status 30))
 (segment (start 236.22 109.22) (end 233.68 109.22) (width 0.508) (layer B.Cu) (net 3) (status 30))
 (segment (start 238.76 109.22) (end 236.22 109.22) (width 0.508) (layer B.Cu) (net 3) (status 30))
 (segment (start 241.3 109.22) (end 238.76 109.22) (width 0.508) (layer B.Cu) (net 3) (status 30))
 (segment (start 243.84 109.22) (end 241.3 109.22) (width 0.508) (layer B.Cu) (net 3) (status 30))
 (segment (start 246.38 109.22) (end 243.84 109.22) (width 0.508) (layer B.Cu) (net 3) (status 30))
 (segment (start 248.92 109.22) (end 246.38 109.22) (width 0.508) (layer B.Cu) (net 3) (status 30))
 (segment (start 251.46 109.22) (end 248.92 109.22) (width 0.508) (layer B.Cu) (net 3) (status 30))
 (segment (start 254 109.22) (end 251.46 109.22) (width 0.508) (layer B.Cu) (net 3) (status 30))
 (segment (start 256.54 109.22) (end 254 109.22) (width 0.508) (layer B.Cu) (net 3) (status 30))
 (segment (start 259.08 109.22) (end 256.54 109.22) (width 0.508) (layer B.Cu) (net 3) (status 30))
 (segment (start 278.11 134.005) (end 280.035 132.08) (width 0.508) (layer B.Cu) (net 3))
 (segment (start 271.78 134.62) (end 272.629999 133.770001) (width 0.254) (layer F.Cu) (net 6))
 (segment (start 272.629999 133.770001) (end 272.629999 120.229999) (width 0.254) (layer F.Cu) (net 6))
 (segment (start 272.629999 120.229999) (end 271.78 119.38) (width 0.254) (layer F.Cu) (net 6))
 (segment (start 215.9 124.46) (end 218.44 121.92) (width 0.508) (layer F.Cu) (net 6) (status 30))
 (segment (start 228.6 121.92) (end 228.6 119.38) (width 0.508) (layer B.Cu) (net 6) (status 20))
 (segment (start 218.44 121.92) (end 228.6 121.92) (width 0.508) (layer B.Cu) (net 6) (status 10))
 (segment (start 256.54 111.76) (end 254 111.76) (width 0.508) (layer B.Cu) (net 6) (status 30))
 (segment (start 246.38 111.76) (end 243.84 111.76) (width 0.508) (layer B.Cu) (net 6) (status 30))
 (segment (start 243.84 111.76) (end 241.3 111.76) (width 0.508) (layer B.Cu) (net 6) (status 30))
 (segment (start 236.22 111.76) (end 233.68 111.76) (width 0.508) (layer B.Cu) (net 6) (status 30))
 (segment (start 233.68 111.76) (end 228.6 111.76) (width 0.508) (layer B.Cu) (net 6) (status 10))
 (segment (start 228.6 111.76) (end 228.6 119.38) (width 0.508) (layer B.Cu) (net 6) (status 20))
 (segment (start 241.3 111.76) (end 238.76 111.76) (width 0.508) (layer B.Cu) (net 6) (status 30))
 (segment (start 236.22 111.76) (end 238.76 111.76) (width 0.508) (layer B.Cu) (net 6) (status 30))
 (segment (start 248.92 111.76) (end 246.38 111.76) (width 0.508) (layer B.Cu) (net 6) (status 30))
 (segment (start 254 111.76) (end 251.46 111.76) (width 0.508) (layer B.Cu) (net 6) (status 30))
 (segment (start 251.46 111.76) (end 248.92 111.76) (width 0.508) (layer B.Cu) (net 6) (status 30))
 (segment (start 259.08 111.76) (end 256.54 111.76) (width 0.508) (layer B.Cu) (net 6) (status 30))
 (segment (start 276.86 119.38) (end 276.86 121.92) (width 0.508) (layer B.Cu) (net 24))
 (segment (start 274.32 121.92) (end 276.86 121.92) (width 0.508) (layer B.Cu) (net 24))
 (segment (start 274.32 137.16) (end 274.32 121.92) (width 0.508) (layer F.Cu) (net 24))
 (segment (start 274.32 137.16) (end 275.61 137.16) (width 0.508) (layer B.Cu) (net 24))
 (segment (start 266.7 137.16) (end 266.7 134.62) (width 0.508) (layer B.Cu) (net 24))
 (segment (start 274.32 137.16) (end 266.7 137.16) (width 0.508) (layer B.Cu) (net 24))
 (via (at 274.32 137.16) (size 0.889) (drill 0.635) (layers F.Cu B.Cu) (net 24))
 (via (at 274.32 121.92) (size 0.889) (drill 0.635) (layers F.Cu B.Cu) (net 24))
 (segment (start 266.7 132.3975) (end 266.7 134.62) (width 0.508) (layer B.Cu) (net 24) (status 30))
 (segment (start 259.08 114.3) (end 259.08 119.38) (width 0.508) (layer B.Cu) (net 29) (status 30))
 (segment (start 256.54 114.3) (end 256.54 119.38) (width 0.508) (layer B.Cu) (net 30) (status 30))
 (segment (start 254 119.38) (end 254 114.3) (width 0.508) (layer B.Cu) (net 31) (status 30))
 (segment (start 251.46 114.3) (end 251.46 119.38) (width 0.508) (layer B.Cu) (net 32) (status 30))
 (segment (start 248.92 114.3) (end 248.92 119.38) (width 0.508) (layer B.Cu) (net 33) (status 30))
 (segment (start 246.38 114.3) (end 246.38 119.38) (width 0.508) (layer B.Cu) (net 34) (status 30))
 (segment (start 243.84 114.3) (end 243.84 119.38) (width 0.508) (layer B.Cu) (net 35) (status 30))
 (segment (start 287.02 109.22) (end 284.48 111.76) (width 0.508) (layer B.Cu) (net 5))
 (segment (start 284.48 111.76) (end 276.86 111.76) (width 0.508) (layer B.Cu) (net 5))
 (segment (start 294.005 109.22) (end 287.02 109.22) (width 0.508) (layer B.Cu) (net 5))
 (segment (start 294.005 109.22) (end 294.005 108.585) (width 0.508) (layer B.Cu) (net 5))
 (segment (start 276.86 127) (end 276.86 124.46) (width 0.508) (layer B.Cu) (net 43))
 (segment (start 276.86 129.54) (end 271.78 129.54) (width 0.508) (layer B.Cu) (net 42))
 (segment (start 246.38 129.54) (end 246.38 130.73) (width 0.508) (layer B.Cu) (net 42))
 (via (at 246.38 129.54) (size 0.889) (drill 0.635) (layers F.Cu B.Cu) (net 42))
 (segment (start 271.78 129.54) (end 246.38 129.54) (width 0.508) (layer F.Cu) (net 42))
 (via (at 271.78 129.54) (size 0.889) (drill 0.635) (layers F.Cu B.Cu) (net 42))
 (segment (start 279.4 127) (end 279.4 118.022) (width 0.508) (layer B.Cu) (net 1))
 (segment (start 279.4 118.022) (end 278.218 116.84) (width 0.508) (layer B.Cu) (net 1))
 (segment (start 278.218 116.84) (end 276.86 116.84) (width 0.508) (layer B.Cu) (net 1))
 (segment (start 281.94 129.54) (end 279.4 127) (width 0.508) (layer B.Cu) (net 1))
 (segment (start 293.37 129.54) (end 281.94 129.54) (width 0.508) (layer B.Cu) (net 1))
 (segment (start 294.005 130.175) (end 293.37 129.54) (width 0.508) (layer B.Cu) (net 1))
 (segment (start 294.005 132.08) (end 294.005 130.175) (width 0.508) (layer B.Cu) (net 1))
 (segment (start 284.48 134.62) (end 287.02 132.08) (width 0.508) (layer B.Cu) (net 2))
 (segment (start 287.02 132.08) (end 290.83 132.08) (width 0.508) (layer B.Cu) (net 2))
 (segment (start 284.48 137.16) (end 284.48 134.62) (width 0.508) (layer B.Cu) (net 2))
 (segment (start 281.94 137.16) (end 281.94 133.35) (width 0.508) (layer B.Cu) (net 4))
 (segment (start 281.94 133.35) (end 283.21 132.08) (width 0.508) (layer B.Cu) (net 4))
 (segment (start 264.16 133.43) (end 264.16 134.62) (width 0.508) (layer B.Cu) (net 23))
 (segment (start 266.7 111.76) (end 269.2 111.76) (width 0.508) (layer B.Cu) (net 44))
 (segment (start 269.2 111.76) (end 269.24 111.72) (width 0.508) (layer B.Cu) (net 44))
 (segment (start 264.16 111.76) (end 266.7 111.76) (width 0.508) (layer B.Cu) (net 44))
 (segment (start 264.16 116.84) (end 264.16 111.76) (width 0.508) (layer F.Cu) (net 44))
 (via (at 264.16 111.76) (size 0.889) (drill 0.635) (layers F.Cu B.Cu) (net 44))
 (segment (start 265.365601 118.045601) (end 264.16 116.84) (width 0.508) (layer F.Cu) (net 44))
 (segment (start 264.16 127) (end 265.365601 125.794399) (width 0.508) (layer F.Cu) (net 44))
 (segment (start 265.365601 125.794399) (end 265.365601 118.045601) (width 0.508) (layer F.Cu) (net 44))
 (via (at 264.16 127) (size 0.889) (drill 0.635) (layers F.Cu B.Cu) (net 44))
 (segment (start 264.16 130.73) (end 264.16 127) (width 0.508) (layer B.Cu) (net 44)))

